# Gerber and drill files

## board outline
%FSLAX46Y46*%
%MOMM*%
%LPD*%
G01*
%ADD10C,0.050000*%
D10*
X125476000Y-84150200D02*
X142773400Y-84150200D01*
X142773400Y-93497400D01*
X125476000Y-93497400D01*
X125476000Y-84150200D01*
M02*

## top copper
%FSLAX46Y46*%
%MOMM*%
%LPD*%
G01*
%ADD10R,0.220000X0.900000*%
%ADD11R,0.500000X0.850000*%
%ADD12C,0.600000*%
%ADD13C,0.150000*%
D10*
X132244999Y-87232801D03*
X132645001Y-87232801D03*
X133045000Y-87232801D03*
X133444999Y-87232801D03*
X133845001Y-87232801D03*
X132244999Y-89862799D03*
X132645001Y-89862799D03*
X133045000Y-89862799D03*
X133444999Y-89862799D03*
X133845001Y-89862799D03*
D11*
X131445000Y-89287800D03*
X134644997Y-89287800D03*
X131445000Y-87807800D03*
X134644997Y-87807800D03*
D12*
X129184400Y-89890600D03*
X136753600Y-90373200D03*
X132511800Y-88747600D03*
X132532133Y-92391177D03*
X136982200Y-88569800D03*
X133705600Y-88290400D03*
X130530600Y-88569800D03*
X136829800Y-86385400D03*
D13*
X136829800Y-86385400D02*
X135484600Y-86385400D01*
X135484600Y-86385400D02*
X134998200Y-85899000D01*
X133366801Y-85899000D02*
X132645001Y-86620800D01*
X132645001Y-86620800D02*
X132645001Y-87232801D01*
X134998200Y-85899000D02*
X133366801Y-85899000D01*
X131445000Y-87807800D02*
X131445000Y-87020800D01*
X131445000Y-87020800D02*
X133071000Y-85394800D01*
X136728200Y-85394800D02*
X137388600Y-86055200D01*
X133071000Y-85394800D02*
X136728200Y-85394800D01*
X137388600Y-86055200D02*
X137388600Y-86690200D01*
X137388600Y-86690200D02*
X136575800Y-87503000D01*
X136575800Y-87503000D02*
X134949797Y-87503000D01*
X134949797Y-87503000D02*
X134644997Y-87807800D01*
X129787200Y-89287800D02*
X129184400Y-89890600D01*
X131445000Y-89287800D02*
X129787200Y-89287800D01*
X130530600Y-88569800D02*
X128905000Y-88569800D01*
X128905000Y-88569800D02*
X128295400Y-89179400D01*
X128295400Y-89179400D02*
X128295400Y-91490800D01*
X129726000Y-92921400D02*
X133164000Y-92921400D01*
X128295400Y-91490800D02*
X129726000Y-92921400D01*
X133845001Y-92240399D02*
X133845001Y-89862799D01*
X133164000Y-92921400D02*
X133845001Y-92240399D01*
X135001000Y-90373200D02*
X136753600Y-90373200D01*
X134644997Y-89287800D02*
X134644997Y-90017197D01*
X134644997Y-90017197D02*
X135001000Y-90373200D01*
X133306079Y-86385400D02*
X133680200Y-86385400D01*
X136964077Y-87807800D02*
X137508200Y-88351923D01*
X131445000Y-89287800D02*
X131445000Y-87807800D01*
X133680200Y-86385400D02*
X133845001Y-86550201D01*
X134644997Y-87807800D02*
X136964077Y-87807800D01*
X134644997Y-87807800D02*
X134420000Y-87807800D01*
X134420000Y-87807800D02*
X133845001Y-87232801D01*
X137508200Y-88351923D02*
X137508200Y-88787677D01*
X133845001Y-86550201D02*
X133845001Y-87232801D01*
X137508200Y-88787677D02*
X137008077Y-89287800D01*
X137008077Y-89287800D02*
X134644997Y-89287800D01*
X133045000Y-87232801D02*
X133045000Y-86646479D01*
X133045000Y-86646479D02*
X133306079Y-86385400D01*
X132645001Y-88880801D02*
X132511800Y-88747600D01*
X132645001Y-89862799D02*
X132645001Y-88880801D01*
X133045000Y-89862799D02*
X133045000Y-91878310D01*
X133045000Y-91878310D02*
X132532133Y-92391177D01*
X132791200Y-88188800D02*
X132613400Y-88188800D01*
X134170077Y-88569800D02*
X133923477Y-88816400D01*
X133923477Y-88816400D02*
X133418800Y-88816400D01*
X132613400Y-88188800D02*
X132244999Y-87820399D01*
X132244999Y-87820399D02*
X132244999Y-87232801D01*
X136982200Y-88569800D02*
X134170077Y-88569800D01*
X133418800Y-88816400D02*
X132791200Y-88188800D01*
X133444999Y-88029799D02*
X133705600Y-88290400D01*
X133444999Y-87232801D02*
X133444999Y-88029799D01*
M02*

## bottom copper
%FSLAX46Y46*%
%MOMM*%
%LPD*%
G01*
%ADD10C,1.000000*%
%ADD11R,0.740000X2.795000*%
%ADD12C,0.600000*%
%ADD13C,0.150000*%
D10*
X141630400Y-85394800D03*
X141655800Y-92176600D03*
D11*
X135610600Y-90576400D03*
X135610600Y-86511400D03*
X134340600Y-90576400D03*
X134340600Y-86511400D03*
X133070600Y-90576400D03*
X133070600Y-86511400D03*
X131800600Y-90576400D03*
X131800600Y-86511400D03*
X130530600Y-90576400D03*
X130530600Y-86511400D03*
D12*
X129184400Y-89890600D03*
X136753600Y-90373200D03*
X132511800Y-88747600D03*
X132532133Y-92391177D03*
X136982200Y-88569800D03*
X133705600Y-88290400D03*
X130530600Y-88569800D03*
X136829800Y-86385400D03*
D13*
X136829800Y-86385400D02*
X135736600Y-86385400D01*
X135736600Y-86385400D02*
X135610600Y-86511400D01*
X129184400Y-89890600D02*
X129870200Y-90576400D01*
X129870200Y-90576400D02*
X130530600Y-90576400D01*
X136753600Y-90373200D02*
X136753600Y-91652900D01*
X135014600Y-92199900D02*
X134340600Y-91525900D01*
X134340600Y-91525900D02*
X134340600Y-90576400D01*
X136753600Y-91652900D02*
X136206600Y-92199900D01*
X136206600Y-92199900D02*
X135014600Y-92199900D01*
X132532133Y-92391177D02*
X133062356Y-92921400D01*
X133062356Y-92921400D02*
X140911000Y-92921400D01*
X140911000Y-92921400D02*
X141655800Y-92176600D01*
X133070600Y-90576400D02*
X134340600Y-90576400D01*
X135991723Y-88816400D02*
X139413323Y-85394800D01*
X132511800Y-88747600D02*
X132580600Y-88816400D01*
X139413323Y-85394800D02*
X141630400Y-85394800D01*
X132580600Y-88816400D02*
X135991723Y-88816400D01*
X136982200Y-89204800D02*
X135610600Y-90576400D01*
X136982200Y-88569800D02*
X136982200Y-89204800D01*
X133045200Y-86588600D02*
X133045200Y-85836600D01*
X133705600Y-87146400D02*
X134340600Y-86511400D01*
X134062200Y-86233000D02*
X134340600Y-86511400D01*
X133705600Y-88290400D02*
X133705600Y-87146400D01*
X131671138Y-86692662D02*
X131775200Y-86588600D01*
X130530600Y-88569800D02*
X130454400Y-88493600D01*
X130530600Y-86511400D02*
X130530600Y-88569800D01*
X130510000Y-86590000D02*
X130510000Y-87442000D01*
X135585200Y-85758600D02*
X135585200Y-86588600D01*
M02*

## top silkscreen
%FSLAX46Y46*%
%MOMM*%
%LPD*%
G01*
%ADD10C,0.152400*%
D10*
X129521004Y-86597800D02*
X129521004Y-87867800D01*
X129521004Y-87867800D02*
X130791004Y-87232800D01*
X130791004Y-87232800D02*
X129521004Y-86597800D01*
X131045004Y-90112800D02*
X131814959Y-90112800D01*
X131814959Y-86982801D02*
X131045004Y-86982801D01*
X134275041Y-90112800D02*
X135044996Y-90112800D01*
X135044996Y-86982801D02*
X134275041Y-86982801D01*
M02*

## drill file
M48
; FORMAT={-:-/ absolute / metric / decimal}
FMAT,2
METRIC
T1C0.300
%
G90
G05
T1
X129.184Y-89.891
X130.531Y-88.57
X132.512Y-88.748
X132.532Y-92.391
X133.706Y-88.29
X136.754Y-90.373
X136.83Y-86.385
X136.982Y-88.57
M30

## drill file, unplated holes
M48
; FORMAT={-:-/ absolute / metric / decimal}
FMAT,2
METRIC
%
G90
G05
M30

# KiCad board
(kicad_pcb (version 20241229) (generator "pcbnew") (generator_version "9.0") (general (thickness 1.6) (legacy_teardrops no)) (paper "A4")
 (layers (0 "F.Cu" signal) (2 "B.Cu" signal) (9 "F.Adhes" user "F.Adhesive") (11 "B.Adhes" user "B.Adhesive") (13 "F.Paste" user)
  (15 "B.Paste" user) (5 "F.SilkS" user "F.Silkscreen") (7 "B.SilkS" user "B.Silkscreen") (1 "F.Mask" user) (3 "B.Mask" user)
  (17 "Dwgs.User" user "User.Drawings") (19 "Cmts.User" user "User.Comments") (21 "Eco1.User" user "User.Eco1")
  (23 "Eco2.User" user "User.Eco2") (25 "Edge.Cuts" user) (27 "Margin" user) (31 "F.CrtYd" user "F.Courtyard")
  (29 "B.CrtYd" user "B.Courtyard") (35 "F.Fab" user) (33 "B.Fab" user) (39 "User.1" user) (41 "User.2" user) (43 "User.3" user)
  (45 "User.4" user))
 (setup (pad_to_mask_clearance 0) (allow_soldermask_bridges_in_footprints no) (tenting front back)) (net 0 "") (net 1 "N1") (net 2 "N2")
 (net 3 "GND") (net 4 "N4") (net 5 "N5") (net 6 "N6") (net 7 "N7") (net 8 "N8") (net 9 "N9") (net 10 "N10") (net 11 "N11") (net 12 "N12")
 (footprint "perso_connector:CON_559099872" (layer "F.Cu") (at 133.045 88.5478)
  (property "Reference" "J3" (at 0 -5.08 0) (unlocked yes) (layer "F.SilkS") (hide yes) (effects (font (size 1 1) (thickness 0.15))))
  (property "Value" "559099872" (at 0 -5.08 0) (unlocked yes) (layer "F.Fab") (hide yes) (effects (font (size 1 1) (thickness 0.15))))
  (fp_line (start -3.523996 -1.95) (end -3.523996 -0.68) (stroke (width 0.1524) (type solid)) (layer "F.SilkS"))
  (fp_line (start -3.523996 -0.68) (end -2.253996 -1.315) (stroke (width 0.1524) (type solid)) (layer "F.SilkS"))
  (fp_line (start -2.253996 -1.315) (end -3.523996 -1.95) (stroke (width 0.1524) (type solid)) (layer "F.SilkS"))
  (fp_line (start -1.999996 1.565) (end -1.230041 1.565) (stroke (width 0.1524) (type solid)) (layer "F.SilkS"))
  (fp_line (start -1.230041 -1.564999) (end -1.999996 -1.564999) (stroke (width 0.1524) (type solid)) (layer "F.SilkS"))
  (fp_line (start 1.230041 1.565) (end 1.999996 1.565) (stroke (width 0.1524) (type solid)) (layer "F.SilkS"))
  (fp_line (start 1.999996 -1.564999) (end 1.230041 -1.564999) (stroke (width 0.1524) (type solid)) (layer "F.SilkS"))
  (pad "1" smd rect (at -0.800001 -1.314999) (size 0.22 0.9) (layers "F.Cu" "F.Mask" "F.Paste") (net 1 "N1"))
  (pad "2" smd rect (at -0.399999 -1.314999) (size 0.22 0.9) (layers "F.Cu" "F.Mask" "F.Paste") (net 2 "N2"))
  (pad "3" smd rect (at 0 -1.314999) (size 0.22 0.9) (layers "F.Cu" "F.Mask" "F.Paste") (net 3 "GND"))
  (pad "4" smd rect (at 0.399999 -1.314999) (size 0.22 0.9) (layers "F.Cu" "F.Mask" "F.Paste") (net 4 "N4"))
  (pad "5" smd rect (at 0.800001 -1.314999) (size 0.22 0.9) (layers "F.Cu" "F.Mask" "F.Paste") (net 3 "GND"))
  (pad "6" smd rect (at -0.800001 1.314999) (size 0.22 0.9) (layers "F.Cu" "F.Mask" "F.Paste") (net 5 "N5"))
  (pad "7" smd rect (at -0.399999 1.314999) (size 0.22 0.9) (layers "F.Cu" "F.Mask" "F.Paste") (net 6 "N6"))
  (pad "8" smd rect (at 0 1.314999) (size 0.22 0.9) (layers "F.Cu" "F.Mask" "F.Paste") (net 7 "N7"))
  (pad "9" smd rect (at 0.399999 1.314999) (size 0.22 0.9) (layers "F.Cu" "F.Mask" "F.Paste") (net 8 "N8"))
  (pad "10" smd rect (at 0.800001 1.314999) (size 0.22 0.9) (layers "F.Cu" "F.Mask" "F.Paste") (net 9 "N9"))
  (pad "P1" smd rect (at -1.6 0.74) (size 0.5 0.85) (layers "F.Cu" "F.Mask" "F.Paste") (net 3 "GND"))
  (pad "P2" smd rect (at 1.599997 0.74) (size 0.5 0.85) (layers "F.Cu" "F.Mask" "F.Paste") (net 3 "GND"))
  (pad "P3" smd rect (at -1.6 -0.74) (size 0.5 0.85) (layers "F.Cu" "F.Mask" "F.Paste") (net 3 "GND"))
  (pad "P4" smd rect (at 1.599997 -0.74) (size 0.5 0.85) (layers "F.Cu" "F.Mask" "F.Paste") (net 3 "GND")))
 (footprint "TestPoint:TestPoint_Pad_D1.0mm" (layer "B.Cu") (at 141.6304 85.3948 180)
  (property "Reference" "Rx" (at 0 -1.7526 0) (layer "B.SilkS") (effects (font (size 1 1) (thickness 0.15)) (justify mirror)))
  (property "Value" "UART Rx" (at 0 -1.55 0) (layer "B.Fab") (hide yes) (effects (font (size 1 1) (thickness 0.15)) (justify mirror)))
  (pad "1" smd circle (at 0 0 180) (size 1 1) (layers "B.Cu" "B.Mask") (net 6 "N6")))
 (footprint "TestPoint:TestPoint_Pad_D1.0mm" (layer "B.Cu") (at 141.6558 92.1766 180)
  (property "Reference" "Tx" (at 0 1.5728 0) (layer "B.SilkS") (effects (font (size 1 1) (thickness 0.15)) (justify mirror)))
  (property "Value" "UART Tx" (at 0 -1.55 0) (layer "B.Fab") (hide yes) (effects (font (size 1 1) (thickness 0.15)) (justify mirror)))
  (pad "1" smd circle (at 0 0 180) (size 1 1) (layers "B.Cu" "B.Mask") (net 7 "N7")))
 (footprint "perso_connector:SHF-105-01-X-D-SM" (layer "B.Cu") (at 133.0706 88.5439 180)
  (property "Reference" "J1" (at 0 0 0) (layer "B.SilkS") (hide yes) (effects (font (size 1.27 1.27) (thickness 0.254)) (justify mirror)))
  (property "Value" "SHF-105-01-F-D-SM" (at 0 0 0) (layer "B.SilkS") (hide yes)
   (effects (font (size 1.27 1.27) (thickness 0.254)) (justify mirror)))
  (pad "1" smd rect (at -2.54 -2.0325 180) (size 0.74 2.795) (layers "B.Cu" "B.Mask" "B.Paste") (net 1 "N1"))
  (pad "2" smd rect (at -2.54 2.0325 180) (size 0.74 2.795) (layers "B.Cu" "B.Mask" "B.Paste") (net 2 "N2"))
  (pad "3" smd rect (at -1.27 -2.0325 180) (size 0.74 2.795) (layers "B.Cu" "B.Mask" "B.Paste") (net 3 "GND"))
  (pad "4" smd rect (at -1.27 2.0325 180) (size 0.74 2.795) (layers "B.Cu" "B.Mask" "B.Paste") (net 4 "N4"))
  (pad "5" smd rect (at 0 -2.0325 180) (size 0.74 2.795) (layers "B.Cu" "B.Mask" "B.Paste") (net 3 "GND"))
  (pad "6" smd rect (at 0 2.0325 180) (size 0.74 2.795) (layers "B.Cu" "B.Mask" "B.Paste") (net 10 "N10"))
  (pad "7" smd rect (at 1.27 -2.0325 180) (size 0.74 2.795) (layers "B.Cu" "B.Mask" "B.Paste") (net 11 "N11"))
  (pad "8" smd rect (at 1.27 2.0325 180) (size 0.74 2.795) (layers "B.Cu" "B.Mask" "B.Paste") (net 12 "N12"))
  (pad "9" smd rect (at 2.54 -2.0325 180) (size 0.74 2.795) (layers "B.Cu" "B.Mask" "B.Paste") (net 3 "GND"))
  (pad "10" smd rect (at 2.54 2.0325 180) (size 0.74 2.795) (layers "B.Cu" "B.Mask" "B.Paste") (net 9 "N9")))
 (gr_rect (start 125.476 84.1502) (end 142.7734 93.4974) (stroke (width 0.05) (type default)) (fill no) (layer "Edge.Cuts"))
 (segment (start 131.445 87.0208) (end 133.071 85.3948) (width 0.15) (layer "F.Cu") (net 3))
 (segment (start 136.5758 87.503) (end 134.949797 87.503) (width 0.15) (layer "F.Cu") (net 3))
 (segment (start 137.3886 86.6902) (end 136.5758 87.503) (width 0.15) (layer "F.Cu") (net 3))
 (segment (start 131.445 89.2878) (end 129.7872 89.2878) (width 0.15) (layer "F.Cu") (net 3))
 (segment (start 137.3886 86.0552) (end 137.3886 86.6902) (width 0.15) (layer "F.Cu") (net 3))
 (segment (start 134.949797 87.503) (end 134.644997 87.8078) (width 0.15) (layer "F.Cu") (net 3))
 (segment (start 134.644997 89.2878) (end 134.644997 90.017197) (width 0.15) (layer "F.Cu") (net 3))
 (segment (start 133.306079 86.3854) (end 133.6802 86.3854) (width 0.15) (layer "F.Cu") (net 3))
 (segment (start 136.964077 87.8078) (end 137.5082 88.351923) (width 0.15) (layer "F.Cu") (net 3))
 (segment (start 131.445 89.2878) (end 131.445 87.8078) (width 0.15) (layer "F.Cu") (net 3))
 (segment (start 131.445 87.8078) (end 131.445 87.0208) (width 0.15) (layer "F.Cu") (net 3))
 (segment (start 129.7872 89.2878) (end 129.1844 89.8906) (width 0.15) (layer "F.Cu") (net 3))
 (segment (start 134.644997 90.017197) (end 135.001 90.3732) (width 0.15) (layer "F.Cu") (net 3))
 (segment (start 133.6802 86.3854) (end 133.845001 86.550201) (width 0.15) (layer "F.Cu") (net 3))
 (segment (start 134.644997 87.8078) (end 136.964077 87.8078) (width 0.15) (layer "F.Cu") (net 3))
 (segment (start 134.644997 87.8078) (end 134.42 87.8078) (width 0.15) (layer "F.Cu") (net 3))
 (segment (start 134.42 87.8078) (end 133.845001 87.232801) (width 0.15) (layer "F.Cu") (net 3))
 (segment (start 133.071 85.3948) (end 136.7282 85.3948) (width 0.15) (layer "F.Cu") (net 3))
 (segment (start 136.7282 85.3948) (end 137.3886 86.0552) (width 0.15) (layer "F.Cu") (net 3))
 (segment (start 137.5082 88.351923) (end 137.5082 88.787677) (width 0.15) (layer "F.Cu") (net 3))
 (segment (start 133.845001 86.550201) (end 133.845001 87.232801) (width 0.15) (layer "F.Cu") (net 3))
 (segment (start 137.5082 88.787677) (end 137.008077 89.2878) (width 0.15) (layer "F.Cu") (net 3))
 (segment (start 135.001 90.3732) (end 136.7536 90.3732) (width 0.15) (layer "F.Cu") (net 3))
 (segment (start 137.008077 89.2878) (end 134.644997 89.2878) (width 0.15) (layer "F.Cu") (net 3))
 (segment (start 133.045 87.232801) (end 133.045 86.646479) (width 0.15) (layer "F.Cu") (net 3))
 (segment (start 133.045 86.646479) (end 133.306079 86.3854) (width 0.15) (layer "F.Cu") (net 3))
 (via (at 129.1844 89.8906) (size 0.6) (drill 0.3) (layers "F.Cu" "B.Cu") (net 3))
 (via (at 136.7536 90.3732) (size 0.6) (drill 0.3) (layers "F.Cu" "B.Cu") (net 3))
 (segment (start 129.1844 89.8906) (end 129.8702 90.5764) (width 0.15) (layer "B.Cu") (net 3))
 (segment (start 133.0706 90.5764) (end 134.3406 90.5764) (width 0.15) (layer "B.Cu") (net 3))
 (segment (start 129.8702 90.5764) (end 130.5306 90.5764) (width 0.15) (layer "B.Cu") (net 3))
 (segment (start 135.0146 92.1999) (end 134.3406 91.5259) (width 0.15) (layer "B.Cu") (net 3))
 (segment (start 136.7536 91.6529) (end 136.2066 92.1999) (width 0.15) (layer "B.Cu") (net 3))
 (segment (start 136.7536 90.3732) (end 136.7536 91.6529) (width 0.15) (layer "B.Cu") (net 3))
 (segment (start 136.2066 92.1999) (end 135.0146 92.1999) (width 0.15) (layer "B.Cu") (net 3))
 (segment (start 134.3406 91.5259) (end 134.3406 90.5764) (width 0.15) (layer "B.Cu") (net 3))
 (segment (start 132.645001 88.880801) (end 132.5118 88.7476) (width 0.15) (layer "F.Cu") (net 6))
 (segment (start 132.645001 89.862799) (end 132.645001 88.880801) (width 0.15) (layer "F.Cu") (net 6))
 (via (at 132.5118 88.7476) (size 0.6) (drill 0.3) (layers "F.Cu" "B.Cu") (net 6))
 (segment (start 135.991723 88.8164) (end 139.413323 85.3948) (width 0.15) (layer "B.Cu") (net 6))
 (segment (start 132.5118 88.7476) (end 132.5806 88.8164) (width 0.15) (layer "B.Cu") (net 6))
 (segment (start 139.413323 85.3948) (end 141.6304 85.3948) (width 0.15) (layer "B.Cu") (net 6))
 (segment (start 132.5806 88.8164) (end 135.991723 88.8164) (width 0.15) (layer "B.Cu") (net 6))
 (segment (start 133.045 89.862799) (end 133.045 91.87831) (width 0.15) (layer "F.Cu") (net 7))
 (segment (start 133.045 91.87831) (end 132.532133 92.391177) (width 0.15) (layer "F.Cu") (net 7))
 (via (at 132.532133 92.391177) (size 0.6) (drill 0.3) (layers "F.Cu" "B.Cu") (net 7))
 (segment (start 133.062356 92.9214) (end 140.911 92.9214) (width 0.15) (layer "B.Cu") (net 7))
 (segment (start 132.532133 92.391177) (end 133.062356 92.9214) (width 0.15) (layer "B.Cu") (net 7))
 (segment (start 140.911 92.9214) (end 141.6558 92.1766) (width 0.15) (layer "B.Cu") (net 7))
 (segment (start 132.7912 88.1888) (end 132.6134 88.1888) (width 0.15) (layer "F.Cu") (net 1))
 (segment (start 134.170077 88.5698) (end 133.923477 88.8164) (width 0.15) (layer "F.Cu") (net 1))
 (segment (start 133.923477 88.8164) (end 133.4188 88.8164) (width 0.15) (layer "F.Cu") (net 1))
 (segment (start 132.6134 88.1888) (end 132.244999 87.820399) (width 0.15) (layer "F.Cu") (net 1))
 (segment (start 132.244999 87.820399) (end 132.244999 87.232801) (width 0.15) (layer "F.Cu") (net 1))
 (segment (start 136.9822 88.5698) (end 134.170077 88.5698) (width 0.15) (layer "F.Cu") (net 1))
 (segment (start 133.4188 88.8164) (end 132.7912 88.1888) (width 0.15) (layer "F.Cu") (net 1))
 (via (at 136.9822 88.5698) (size 0.6) (drill 0.3) (layers "F.Cu" "B.Cu") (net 1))
 (segment (start 136.9822 89.2048) (end 135.6106 90.5764) (width 0.15) (layer "B.Cu") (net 1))
 (segment (start 136.9822 88.5698) (end 136.9822 89.2048) (width 0.15) (layer "B.Cu") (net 1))
 (segment (start 133.0452 86.5886) (end 133.0452 85.8366) (width 0.15) (layer "B.Cu") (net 10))
 (segment (start 133.444999 88.029799) (end 133.7056 88.2904) (width 0.15) (layer "F.Cu") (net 4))
 (segment (start 133.444999 87.232801) (end 133.444999 88.029799) (width 0.15) (layer "F.Cu") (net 4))
 (via (at 133.7056 88.2904) (size 0.6) (drill 0.3) (layers "F.Cu" "B.Cu") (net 4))
 (segment (start 133.7056 87.1464) (end 134.3406 86.5114) (width 0.15) (layer "B.Cu") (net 4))
 (segment (start 134.0622 86.233) (end 134.3406 86.5114) (width 0.15) (layer "B.Cu") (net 4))
 (segment (start 133.7056 88.2904) (end 133.7056 87.1464) (width 0.15) (layer "B.Cu") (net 4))
 (segment (start 131.671138 86.692662) (end 131.7752 86.5886) (width 0.15) (layer "B.Cu") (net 12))
 (segment (start 128.905 88.5698) (end 128.2954 89.1794) (width 0.15) (layer "F.Cu") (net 9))
 (segment (start 129.726 92.9214) (end 133.164 92.9214) (width 0.15) (layer "F.Cu") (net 9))
 (segment (start 128.2954 89.1794) (end 128.2954 91.4908) (width 0.15) (layer "F.Cu") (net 9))
 (segment (start 133.845001 92.240399) (end 133.845001 89.862799) (width 0.15) (layer "F.Cu") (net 9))
 (segment (start 130.5306 88.5698) (end 128.905 88.5698) (width 0.15) (layer "F.Cu") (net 9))
 (segment (start 133.164 92.9214) (end 133.845001 92.240399) (width 0.15) (layer "F.Cu") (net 9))
 (segment (start 128.2954 91.4908) (end 129.726 92.9214) (width 0.15) (layer "F.Cu") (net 9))
 (via (at 130.5306 88.5698) (size 0.6) (drill 0.3) (layers "F.Cu" "B.Cu") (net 9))
 (segment (start 130.5306 88.5698) (end 130.4544 88.4936) (width 0.15) (layer "B.Cu") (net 9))
 (segment (start 130.5306 86.5114) (end 130.5306 88.5698) (width 0.15) (layer "B.Cu") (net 9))
 (segment (start 130.51 86.59) (end 130.51 87.442) (width 0.15) (layer "B.Cu") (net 9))
 (segment (start 136.8298 86.3854) (end 135.4846 86.3854) (width 0.15) (layer "F.Cu") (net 2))
 (segment (start 133.366801 85.899) (end 132.645001 86.6208) (width 0.15) (layer "F.Cu") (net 2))
 (segment (start 132.645001 86.6208) (end 132.645001 87.232801) (width 0.15) (layer "F.Cu") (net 2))
 (segment (start 135.4846 86.3854) (end 134.9982 85.899) (width 0.15) (layer "F.Cu") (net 2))
 (segment (start 134.9982 85.899) (end 133.366801 85.899) (width 0.15) (layer "F.Cu") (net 2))
 (via (at 136.8298 86.3854) (size 0.6) (drill 0.3) (layers "F.Cu" "B.Cu") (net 2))
 (segment (start 136.8298 86.3854) (end 135.7366 86.3854) (width 0.15) (layer "B.Cu") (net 2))
 (segment (start 135.7366 86.3854) (end 135.6106 86.5114) (width 0.15) (layer "B.Cu") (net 2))
 (segment (start 135.5852 85.7586) (end 135.5852 86.5886) (width 0.15) (layer "B.Cu") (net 2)))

